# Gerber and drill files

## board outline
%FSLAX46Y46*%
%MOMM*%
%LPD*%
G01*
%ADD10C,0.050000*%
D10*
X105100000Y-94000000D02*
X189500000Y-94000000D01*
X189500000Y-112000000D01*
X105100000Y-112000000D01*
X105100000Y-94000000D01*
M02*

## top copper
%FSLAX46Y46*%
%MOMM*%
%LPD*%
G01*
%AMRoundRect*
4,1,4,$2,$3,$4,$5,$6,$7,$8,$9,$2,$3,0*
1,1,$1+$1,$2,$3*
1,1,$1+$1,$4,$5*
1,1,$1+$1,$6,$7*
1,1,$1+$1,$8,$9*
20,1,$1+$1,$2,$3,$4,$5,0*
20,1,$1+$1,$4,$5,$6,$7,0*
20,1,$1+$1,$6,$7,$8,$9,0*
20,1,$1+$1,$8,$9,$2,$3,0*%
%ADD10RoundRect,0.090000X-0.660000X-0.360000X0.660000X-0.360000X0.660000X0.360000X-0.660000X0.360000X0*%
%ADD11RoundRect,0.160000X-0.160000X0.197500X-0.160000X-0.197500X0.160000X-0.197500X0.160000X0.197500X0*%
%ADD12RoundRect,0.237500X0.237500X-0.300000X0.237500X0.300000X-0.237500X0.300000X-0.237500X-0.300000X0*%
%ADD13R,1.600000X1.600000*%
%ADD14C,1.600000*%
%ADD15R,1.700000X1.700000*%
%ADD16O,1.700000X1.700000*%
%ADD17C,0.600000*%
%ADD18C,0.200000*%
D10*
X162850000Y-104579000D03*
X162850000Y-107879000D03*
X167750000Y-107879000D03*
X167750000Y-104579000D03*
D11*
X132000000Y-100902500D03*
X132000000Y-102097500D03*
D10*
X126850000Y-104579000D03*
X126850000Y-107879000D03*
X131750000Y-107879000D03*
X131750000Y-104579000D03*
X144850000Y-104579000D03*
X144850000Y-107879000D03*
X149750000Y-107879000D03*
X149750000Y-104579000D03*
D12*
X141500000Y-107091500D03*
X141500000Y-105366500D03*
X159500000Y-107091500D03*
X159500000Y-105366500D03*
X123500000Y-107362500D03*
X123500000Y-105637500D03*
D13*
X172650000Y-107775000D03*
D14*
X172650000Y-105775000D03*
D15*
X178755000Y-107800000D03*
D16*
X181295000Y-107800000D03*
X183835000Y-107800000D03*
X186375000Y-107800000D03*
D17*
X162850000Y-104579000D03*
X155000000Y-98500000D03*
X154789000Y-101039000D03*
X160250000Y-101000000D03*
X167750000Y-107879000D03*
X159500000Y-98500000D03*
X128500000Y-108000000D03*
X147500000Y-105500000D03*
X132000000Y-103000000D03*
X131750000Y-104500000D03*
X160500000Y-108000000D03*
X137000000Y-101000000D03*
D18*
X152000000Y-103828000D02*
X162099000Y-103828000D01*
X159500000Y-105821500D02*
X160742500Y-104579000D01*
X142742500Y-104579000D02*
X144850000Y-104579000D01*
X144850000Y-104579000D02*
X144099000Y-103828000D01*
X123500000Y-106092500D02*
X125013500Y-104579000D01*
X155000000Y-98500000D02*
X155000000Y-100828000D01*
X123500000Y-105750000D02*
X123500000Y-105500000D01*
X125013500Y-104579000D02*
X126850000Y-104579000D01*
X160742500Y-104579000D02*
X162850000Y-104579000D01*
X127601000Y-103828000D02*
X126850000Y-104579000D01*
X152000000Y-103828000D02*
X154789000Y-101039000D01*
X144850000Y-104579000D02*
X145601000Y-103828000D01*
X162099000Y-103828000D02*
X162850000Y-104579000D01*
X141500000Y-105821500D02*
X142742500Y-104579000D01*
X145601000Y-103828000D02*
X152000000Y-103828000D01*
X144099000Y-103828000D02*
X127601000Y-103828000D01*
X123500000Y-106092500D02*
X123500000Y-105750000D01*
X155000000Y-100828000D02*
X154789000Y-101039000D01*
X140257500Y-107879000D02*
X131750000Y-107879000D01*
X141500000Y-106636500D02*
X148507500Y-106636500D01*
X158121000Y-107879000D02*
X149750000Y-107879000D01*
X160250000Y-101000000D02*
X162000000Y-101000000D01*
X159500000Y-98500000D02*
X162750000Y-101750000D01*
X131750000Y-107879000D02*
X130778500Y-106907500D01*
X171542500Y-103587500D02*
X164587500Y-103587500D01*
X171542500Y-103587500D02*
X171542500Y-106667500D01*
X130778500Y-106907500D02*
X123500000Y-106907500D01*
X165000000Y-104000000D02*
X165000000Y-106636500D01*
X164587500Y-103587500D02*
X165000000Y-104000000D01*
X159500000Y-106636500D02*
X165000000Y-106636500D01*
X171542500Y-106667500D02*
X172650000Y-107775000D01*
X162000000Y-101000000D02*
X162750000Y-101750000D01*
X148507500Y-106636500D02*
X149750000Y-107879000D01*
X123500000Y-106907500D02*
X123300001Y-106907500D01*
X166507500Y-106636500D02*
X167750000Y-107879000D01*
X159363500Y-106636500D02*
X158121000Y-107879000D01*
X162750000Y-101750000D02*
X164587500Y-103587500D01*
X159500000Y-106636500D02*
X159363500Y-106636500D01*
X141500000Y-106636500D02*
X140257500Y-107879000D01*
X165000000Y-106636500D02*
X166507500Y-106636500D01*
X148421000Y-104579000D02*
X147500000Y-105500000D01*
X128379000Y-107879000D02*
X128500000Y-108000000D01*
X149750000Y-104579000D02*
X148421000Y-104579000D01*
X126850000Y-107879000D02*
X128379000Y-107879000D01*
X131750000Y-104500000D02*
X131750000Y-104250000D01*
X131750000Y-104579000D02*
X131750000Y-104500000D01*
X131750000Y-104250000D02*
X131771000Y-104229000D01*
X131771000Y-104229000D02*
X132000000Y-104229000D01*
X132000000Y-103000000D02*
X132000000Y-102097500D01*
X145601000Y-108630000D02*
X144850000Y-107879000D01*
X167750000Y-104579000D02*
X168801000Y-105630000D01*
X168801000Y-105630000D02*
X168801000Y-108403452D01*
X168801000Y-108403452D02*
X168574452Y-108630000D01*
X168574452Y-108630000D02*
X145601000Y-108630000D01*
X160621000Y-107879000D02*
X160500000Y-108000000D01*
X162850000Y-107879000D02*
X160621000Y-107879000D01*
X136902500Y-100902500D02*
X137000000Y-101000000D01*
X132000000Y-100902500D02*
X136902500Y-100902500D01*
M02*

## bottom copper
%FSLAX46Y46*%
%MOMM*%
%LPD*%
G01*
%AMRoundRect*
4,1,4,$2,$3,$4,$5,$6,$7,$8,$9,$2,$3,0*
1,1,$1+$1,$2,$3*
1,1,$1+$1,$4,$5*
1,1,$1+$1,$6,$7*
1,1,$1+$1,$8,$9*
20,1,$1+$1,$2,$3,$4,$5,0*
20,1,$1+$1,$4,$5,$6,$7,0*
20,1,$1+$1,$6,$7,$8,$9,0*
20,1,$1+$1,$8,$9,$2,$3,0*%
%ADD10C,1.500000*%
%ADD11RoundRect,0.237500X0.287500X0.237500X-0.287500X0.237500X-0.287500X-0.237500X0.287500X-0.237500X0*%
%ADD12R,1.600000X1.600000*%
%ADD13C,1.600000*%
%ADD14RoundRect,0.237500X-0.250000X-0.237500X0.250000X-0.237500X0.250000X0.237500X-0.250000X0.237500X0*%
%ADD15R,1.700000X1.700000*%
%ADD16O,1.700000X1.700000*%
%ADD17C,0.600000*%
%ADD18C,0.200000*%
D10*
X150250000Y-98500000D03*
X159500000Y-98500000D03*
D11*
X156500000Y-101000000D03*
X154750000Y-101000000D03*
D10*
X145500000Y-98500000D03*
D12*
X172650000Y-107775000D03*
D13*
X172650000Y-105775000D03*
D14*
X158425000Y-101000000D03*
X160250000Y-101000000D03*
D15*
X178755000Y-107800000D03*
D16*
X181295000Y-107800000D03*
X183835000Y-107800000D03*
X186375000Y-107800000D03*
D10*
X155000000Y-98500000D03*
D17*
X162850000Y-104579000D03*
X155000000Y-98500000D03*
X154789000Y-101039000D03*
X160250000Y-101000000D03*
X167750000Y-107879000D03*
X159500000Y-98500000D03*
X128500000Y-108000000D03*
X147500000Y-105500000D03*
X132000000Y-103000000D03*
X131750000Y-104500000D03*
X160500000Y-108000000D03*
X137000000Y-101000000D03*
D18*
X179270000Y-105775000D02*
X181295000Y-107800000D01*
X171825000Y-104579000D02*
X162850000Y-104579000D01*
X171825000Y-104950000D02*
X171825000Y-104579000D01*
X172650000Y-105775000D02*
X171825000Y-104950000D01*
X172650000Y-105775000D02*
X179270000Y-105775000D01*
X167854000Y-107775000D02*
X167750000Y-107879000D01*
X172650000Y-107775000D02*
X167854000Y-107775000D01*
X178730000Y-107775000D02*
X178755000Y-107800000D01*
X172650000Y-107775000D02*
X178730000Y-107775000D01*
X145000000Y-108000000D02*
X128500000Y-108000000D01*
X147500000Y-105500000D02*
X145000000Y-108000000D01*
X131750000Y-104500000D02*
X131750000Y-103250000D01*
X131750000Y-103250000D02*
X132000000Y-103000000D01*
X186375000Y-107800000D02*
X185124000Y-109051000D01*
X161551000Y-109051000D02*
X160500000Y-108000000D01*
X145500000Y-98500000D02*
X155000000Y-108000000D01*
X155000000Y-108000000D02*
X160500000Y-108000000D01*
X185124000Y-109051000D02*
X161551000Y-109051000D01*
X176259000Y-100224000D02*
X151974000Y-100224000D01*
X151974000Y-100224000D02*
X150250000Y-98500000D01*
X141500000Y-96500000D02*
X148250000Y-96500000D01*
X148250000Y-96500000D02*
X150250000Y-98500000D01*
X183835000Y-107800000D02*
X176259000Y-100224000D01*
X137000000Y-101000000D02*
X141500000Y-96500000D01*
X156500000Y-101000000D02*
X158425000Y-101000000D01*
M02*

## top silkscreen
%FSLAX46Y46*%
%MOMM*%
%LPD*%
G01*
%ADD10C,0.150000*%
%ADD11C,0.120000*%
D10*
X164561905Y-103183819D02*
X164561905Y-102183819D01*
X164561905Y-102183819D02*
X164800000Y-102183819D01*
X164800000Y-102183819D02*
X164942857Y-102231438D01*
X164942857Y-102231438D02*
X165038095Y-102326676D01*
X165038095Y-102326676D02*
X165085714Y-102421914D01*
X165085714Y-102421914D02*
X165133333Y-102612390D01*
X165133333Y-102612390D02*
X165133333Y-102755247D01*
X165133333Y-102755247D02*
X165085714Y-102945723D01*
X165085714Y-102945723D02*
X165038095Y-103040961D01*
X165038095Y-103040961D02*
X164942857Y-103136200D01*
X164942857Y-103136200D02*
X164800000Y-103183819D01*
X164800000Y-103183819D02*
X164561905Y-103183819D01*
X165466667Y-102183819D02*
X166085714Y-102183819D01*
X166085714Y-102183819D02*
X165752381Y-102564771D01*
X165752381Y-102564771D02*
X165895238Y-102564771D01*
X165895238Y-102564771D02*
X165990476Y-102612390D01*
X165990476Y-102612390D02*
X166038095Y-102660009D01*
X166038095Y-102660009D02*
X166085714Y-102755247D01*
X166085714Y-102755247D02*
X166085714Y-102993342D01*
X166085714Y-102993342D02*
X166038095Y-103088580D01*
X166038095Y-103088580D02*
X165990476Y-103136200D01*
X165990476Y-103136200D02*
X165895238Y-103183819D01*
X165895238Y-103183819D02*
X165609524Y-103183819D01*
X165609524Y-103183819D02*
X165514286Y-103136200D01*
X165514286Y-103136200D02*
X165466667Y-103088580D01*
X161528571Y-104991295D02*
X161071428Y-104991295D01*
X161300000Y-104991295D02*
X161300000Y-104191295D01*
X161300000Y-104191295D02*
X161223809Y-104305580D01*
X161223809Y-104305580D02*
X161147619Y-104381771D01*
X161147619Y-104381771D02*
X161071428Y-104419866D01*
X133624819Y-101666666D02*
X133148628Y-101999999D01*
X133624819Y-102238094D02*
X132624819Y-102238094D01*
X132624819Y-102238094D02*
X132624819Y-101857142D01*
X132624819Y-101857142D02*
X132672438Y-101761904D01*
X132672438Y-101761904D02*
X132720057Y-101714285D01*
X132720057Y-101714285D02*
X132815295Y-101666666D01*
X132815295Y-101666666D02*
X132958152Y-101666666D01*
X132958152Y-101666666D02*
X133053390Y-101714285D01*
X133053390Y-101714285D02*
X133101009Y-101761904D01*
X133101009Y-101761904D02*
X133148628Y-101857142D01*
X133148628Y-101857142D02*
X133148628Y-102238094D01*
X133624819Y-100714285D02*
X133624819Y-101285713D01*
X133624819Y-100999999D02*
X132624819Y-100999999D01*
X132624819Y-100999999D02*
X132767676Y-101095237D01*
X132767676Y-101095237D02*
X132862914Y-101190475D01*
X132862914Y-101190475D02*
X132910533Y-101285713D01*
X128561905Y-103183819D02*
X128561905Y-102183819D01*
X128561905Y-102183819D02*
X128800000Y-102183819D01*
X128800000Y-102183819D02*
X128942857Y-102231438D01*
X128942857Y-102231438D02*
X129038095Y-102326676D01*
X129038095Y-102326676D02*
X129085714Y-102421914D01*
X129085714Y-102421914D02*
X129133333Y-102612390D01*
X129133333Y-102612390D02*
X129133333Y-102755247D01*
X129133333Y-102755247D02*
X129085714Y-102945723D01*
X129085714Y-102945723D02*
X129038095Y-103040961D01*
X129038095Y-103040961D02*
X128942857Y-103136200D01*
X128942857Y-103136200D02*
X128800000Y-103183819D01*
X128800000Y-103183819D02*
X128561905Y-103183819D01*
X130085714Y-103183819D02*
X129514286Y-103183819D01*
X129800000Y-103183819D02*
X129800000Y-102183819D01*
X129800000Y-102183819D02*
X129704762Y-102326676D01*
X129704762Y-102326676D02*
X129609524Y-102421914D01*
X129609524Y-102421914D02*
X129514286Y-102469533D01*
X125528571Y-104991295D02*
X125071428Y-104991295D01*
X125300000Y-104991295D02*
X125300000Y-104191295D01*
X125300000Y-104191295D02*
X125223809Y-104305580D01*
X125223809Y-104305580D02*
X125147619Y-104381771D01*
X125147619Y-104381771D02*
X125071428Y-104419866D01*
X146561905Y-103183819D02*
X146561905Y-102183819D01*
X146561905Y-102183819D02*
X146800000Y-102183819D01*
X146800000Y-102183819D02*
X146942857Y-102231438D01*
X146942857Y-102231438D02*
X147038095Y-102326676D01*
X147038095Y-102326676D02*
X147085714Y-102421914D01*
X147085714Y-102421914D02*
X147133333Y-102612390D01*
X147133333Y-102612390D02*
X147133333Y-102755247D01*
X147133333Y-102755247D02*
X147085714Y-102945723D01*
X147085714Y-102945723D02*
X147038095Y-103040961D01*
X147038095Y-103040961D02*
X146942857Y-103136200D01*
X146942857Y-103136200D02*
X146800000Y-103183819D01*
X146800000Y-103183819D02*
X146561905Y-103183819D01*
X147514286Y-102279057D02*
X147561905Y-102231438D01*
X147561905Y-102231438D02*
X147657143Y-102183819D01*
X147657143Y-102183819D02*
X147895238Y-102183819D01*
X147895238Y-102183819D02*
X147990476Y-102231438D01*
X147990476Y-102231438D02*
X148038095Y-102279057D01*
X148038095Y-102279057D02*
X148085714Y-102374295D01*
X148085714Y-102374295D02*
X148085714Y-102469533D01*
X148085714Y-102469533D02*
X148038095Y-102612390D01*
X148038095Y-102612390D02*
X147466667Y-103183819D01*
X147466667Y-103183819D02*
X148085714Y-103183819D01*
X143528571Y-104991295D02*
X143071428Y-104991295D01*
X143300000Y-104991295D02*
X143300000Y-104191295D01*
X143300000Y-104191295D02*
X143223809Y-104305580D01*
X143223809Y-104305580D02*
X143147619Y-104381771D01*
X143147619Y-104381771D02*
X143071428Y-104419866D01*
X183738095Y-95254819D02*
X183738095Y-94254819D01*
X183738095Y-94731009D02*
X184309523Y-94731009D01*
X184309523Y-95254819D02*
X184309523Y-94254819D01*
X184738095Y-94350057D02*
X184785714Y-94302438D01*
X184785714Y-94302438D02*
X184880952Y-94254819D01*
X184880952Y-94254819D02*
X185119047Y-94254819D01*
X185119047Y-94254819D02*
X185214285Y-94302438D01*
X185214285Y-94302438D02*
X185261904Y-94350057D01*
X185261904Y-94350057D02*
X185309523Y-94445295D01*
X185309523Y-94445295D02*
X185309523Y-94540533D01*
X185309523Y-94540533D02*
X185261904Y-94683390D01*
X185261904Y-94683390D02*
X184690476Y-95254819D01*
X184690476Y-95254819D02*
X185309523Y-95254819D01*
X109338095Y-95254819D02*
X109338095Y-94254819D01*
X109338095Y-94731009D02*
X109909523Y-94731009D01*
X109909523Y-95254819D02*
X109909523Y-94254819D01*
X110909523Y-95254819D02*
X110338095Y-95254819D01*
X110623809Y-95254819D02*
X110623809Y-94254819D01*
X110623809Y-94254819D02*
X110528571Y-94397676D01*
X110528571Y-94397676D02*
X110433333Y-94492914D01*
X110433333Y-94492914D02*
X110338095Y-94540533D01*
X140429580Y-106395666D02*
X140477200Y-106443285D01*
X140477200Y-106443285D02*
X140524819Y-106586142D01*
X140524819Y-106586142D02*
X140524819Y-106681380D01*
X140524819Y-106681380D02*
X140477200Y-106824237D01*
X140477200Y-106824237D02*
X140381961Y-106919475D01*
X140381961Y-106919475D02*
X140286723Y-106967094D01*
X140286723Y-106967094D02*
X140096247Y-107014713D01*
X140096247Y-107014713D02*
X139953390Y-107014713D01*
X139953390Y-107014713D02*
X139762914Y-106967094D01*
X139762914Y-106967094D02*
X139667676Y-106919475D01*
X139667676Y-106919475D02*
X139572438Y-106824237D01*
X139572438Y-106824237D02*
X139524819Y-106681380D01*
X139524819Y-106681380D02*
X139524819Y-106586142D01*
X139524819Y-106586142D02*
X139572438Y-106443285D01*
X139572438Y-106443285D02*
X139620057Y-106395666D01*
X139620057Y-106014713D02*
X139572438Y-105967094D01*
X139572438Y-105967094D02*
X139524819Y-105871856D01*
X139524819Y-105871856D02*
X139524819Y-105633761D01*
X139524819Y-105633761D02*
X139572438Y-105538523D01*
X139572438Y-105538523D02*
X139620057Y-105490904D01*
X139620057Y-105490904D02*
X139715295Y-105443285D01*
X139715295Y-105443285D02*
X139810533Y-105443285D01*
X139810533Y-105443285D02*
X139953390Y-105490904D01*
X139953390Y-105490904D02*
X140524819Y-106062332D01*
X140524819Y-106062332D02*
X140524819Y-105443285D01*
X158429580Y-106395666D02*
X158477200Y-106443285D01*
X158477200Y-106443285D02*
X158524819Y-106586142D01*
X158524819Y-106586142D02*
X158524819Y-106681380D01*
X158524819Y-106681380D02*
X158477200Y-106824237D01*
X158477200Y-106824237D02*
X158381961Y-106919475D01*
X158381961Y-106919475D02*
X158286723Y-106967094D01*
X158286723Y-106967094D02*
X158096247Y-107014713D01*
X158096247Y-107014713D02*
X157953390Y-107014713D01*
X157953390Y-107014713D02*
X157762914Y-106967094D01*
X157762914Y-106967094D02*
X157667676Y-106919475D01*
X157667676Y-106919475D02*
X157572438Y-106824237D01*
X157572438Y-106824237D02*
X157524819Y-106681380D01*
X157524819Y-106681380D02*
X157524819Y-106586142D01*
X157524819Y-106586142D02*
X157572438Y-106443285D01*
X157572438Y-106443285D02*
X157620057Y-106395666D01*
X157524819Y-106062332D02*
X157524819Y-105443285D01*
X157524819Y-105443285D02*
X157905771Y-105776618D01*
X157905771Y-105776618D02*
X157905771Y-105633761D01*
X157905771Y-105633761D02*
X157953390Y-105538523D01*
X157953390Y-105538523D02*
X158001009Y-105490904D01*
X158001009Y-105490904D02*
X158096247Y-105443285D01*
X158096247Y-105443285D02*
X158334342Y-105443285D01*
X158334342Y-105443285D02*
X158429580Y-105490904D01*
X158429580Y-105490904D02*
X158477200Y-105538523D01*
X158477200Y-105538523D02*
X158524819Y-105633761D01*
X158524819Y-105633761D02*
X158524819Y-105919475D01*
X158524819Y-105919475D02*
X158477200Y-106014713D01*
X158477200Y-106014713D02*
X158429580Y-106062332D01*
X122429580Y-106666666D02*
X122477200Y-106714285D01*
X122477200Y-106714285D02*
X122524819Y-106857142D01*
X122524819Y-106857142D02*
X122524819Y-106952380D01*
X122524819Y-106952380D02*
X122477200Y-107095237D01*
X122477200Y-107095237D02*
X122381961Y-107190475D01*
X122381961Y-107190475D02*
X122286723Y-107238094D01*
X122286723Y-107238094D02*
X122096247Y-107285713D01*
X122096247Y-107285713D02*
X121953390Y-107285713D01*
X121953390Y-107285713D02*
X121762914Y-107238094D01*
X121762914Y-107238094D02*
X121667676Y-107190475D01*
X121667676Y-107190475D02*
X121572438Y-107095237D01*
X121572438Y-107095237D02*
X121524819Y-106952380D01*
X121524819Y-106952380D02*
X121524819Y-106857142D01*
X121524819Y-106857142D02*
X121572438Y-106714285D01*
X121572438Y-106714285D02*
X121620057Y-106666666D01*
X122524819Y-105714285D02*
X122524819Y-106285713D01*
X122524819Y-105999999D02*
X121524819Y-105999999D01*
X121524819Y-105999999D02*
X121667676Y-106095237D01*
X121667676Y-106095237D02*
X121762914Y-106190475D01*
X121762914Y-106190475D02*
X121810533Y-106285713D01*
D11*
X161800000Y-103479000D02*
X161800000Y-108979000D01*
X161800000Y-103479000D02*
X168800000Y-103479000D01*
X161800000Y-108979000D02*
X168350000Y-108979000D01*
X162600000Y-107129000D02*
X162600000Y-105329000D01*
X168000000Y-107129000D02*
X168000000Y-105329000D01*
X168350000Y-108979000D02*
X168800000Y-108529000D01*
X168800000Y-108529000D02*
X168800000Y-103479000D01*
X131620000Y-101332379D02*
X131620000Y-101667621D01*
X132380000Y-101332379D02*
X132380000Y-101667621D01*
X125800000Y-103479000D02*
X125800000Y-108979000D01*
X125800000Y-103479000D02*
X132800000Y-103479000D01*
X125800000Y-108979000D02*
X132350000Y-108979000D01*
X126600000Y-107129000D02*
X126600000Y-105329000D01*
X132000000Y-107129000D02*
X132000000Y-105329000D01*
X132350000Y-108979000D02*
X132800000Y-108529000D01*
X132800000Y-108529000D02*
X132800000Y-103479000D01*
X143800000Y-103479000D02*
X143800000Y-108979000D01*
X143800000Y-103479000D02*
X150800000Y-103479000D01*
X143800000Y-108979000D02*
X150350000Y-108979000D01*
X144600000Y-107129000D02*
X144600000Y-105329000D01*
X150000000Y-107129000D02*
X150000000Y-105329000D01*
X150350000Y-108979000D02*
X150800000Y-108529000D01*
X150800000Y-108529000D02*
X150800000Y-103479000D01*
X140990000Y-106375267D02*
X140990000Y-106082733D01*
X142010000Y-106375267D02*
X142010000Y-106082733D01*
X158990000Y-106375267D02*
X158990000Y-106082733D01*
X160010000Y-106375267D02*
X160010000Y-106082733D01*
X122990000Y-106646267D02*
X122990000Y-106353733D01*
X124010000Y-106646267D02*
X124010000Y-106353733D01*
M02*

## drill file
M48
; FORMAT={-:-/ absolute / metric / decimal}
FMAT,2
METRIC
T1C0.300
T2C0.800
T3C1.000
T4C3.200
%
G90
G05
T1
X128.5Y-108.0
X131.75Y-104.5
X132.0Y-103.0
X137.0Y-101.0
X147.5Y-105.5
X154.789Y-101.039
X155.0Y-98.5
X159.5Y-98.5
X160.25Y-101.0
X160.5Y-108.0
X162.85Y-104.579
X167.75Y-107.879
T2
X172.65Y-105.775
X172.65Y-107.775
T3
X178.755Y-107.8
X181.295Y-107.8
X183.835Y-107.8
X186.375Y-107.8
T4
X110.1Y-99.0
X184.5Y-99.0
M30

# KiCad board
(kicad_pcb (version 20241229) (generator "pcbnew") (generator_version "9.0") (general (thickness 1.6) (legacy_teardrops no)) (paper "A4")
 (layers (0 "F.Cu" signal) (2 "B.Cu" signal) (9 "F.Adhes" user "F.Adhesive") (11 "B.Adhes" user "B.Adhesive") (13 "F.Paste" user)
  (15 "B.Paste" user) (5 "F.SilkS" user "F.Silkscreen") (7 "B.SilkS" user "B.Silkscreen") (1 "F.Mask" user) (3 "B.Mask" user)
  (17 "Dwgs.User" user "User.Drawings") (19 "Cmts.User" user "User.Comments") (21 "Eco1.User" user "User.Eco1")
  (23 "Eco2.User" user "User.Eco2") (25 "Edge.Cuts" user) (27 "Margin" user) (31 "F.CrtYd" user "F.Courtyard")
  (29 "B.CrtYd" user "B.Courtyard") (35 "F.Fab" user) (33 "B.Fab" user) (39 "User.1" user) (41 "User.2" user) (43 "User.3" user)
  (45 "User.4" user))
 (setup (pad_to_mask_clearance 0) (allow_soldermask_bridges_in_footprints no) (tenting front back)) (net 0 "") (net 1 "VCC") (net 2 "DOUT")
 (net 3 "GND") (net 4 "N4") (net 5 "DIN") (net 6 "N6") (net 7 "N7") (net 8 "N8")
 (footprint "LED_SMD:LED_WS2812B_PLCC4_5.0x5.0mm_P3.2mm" (layer "F.Cu") (at 165.3 106.229)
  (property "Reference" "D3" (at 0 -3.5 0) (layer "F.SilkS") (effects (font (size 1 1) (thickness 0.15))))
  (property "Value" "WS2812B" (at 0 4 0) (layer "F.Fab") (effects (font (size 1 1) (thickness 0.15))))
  (fp_line (start -3.5 -2.75) (end -3.5 2.75) (stroke (width 0.12) (type default)) (layer "F.SilkS"))
  (fp_line (start -3.5 -2.75) (end 3.5 -2.75) (stroke (width 0.12) (type solid)) (layer "F.SilkS"))
  (fp_line (start -3.5 2.75) (end 3.05 2.75) (stroke (width 0.12) (type solid)) (layer "F.SilkS"))
  (fp_line (start -2.7 0.9) (end -2.7 -0.9) (stroke (width 0.12) (type default)) (layer "F.SilkS"))
  (fp_line (start 2.7 0.9) (end 2.7 -0.9) (stroke (width 0.12) (type default)) (layer "F.SilkS"))
  (fp_line (start 3.05 2.75) (end 3.5 2.3) (stroke (width 0.12) (type default)) (layer "F.SilkS"))
  (fp_line (start 3.5 2.3) (end 3.5 -2.75) (stroke (width 0.12) (type default)) (layer "F.SilkS"))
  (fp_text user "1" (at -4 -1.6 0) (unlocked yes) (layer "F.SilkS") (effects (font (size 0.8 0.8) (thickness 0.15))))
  (pad "1" smd roundrect (at -2.45 -1.65) (size 1.5 0.9) (layers "F.Cu" "F.Mask" "F.Paste") (roundrect_rratio 0.1) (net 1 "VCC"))
  (pad "2" smd roundrect (at -2.45 1.65) (size 1.5 0.9) (layers "F.Cu" "F.Mask" "F.Paste") (roundrect_rratio 0.1) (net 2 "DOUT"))
  (pad "3" smd roundrect (at 2.45 1.65) (size 1.5 0.9) (layers "F.Cu" "F.Mask" "F.Paste") (roundrect_rratio 0.1) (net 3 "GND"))
  (pad "4" smd roundrect (at 2.45 -1.65) (size 1.5 0.9) (layers "F.Cu" "F.Mask" "F.Paste") (roundrect_rratio 0.1) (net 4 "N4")))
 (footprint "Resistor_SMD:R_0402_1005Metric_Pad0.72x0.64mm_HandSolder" (layer "F.Cu") (at 132 101.5 -90)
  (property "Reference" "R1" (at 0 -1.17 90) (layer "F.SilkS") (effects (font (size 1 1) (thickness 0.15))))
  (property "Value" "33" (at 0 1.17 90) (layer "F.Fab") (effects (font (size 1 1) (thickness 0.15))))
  (fp_line (start -0.167621 0.38) (end 0.167621 0.38) (stroke (width 0.12) (type solid)) (layer "F.SilkS"))
  (fp_line (start -0.167621 -0.38) (end 0.167621 -0.38) (stroke (width 0.12) (type solid)) (layer "F.SilkS"))
  (pad "1" smd roundrect (at -0.5975 0 270) (size 0.715 0.64) (layers "F.Cu" "F.Mask" "F.Paste") (roundrect_rratio 0.25) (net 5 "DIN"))
  (pad "2" smd roundrect (at 0.5975 0 270) (size 0.715 0.64) (layers "F.Cu" "F.Mask" "F.Paste") (roundrect_rratio 0.25) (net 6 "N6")))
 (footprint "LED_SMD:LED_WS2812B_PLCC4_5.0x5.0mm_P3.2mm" (layer "F.Cu") (at 129.3 106.229)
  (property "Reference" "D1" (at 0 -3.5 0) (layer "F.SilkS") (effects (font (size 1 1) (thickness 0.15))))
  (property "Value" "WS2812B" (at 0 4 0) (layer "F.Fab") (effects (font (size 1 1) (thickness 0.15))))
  (fp_line (start -3.5 -2.75) (end -3.5 2.75) (stroke (width 0.12) (type default)) (layer "F.SilkS"))
  (fp_line (start -3.5 -2.75) (end 3.5 -2.75) (stroke (width 0.12) (type solid)) (layer "F.SilkS"))
  (fp_line (start -3.5 2.75) (end 3.05 2.75) (stroke (width 0.12) (type solid)) (layer "F.SilkS"))
  (fp_line (start -2.7 0.9) (end -2.7 -0.9) (stroke (width 0.12) (type default)) (layer "F.SilkS"))
  (fp_line (start 2.7 0.9) (end 2.7 -0.9) (stroke (width 0.12) (type default)) (layer "F.SilkS"))
  (fp_line (start 3.05 2.75) (end 3.5 2.3) (stroke (width 0.12) (type default)) (layer "F.SilkS"))
  (fp_line (start 3.5 2.3) (end 3.5 -2.75) (stroke (width 0.12) (type default)) (layer "F.SilkS"))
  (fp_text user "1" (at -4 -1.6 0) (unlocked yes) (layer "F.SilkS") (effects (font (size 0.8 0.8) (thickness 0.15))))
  (pad "1" smd roundrect (at -2.45 -1.65) (size 1.5 0.9) (layers "F.Cu" "F.Mask" "F.Paste") (roundrect_rratio 0.1) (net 1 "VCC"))
  (pad "2" smd roundrect (at -2.45 1.65) (size 1.5 0.9) (layers "F.Cu" "F.Mask" "F.Paste") (roundrect_rratio 0.1) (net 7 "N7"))
  (pad "3" smd roundrect (at 2.45 1.65) (size 1.5 0.9) (layers "F.Cu" "F.Mask" "F.Paste") (roundrect_rratio 0.1) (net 3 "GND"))
  (pad "4" smd roundrect (at 2.45 -1.65) (size 1.5 0.9) (layers "F.Cu" "F.Mask" "F.Paste") (roundrect_rratio 0.1) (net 6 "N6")))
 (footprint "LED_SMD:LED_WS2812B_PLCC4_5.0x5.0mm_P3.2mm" (layer "F.Cu") (at 147.3 106.229)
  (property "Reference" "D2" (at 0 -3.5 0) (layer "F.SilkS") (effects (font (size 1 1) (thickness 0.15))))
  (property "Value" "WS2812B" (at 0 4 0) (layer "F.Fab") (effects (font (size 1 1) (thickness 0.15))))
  (fp_line (start -3.5 -2.75) (end -3.5 2.75) (stroke (width 0.12) (type default)) (layer "F.SilkS"))
  (fp_line (start -3.5 -2.75) (end 3.5 -2.75) (stroke (width 0.12) (type solid)) (layer "F.SilkS"))
  (fp_line (start -3.5 2.75) (end 3.05 2.75) (stroke (width 0.12) (type solid)) (layer "F.SilkS"))
  (fp_line (start -2.7 0.9) (end -2.7 -0.9) (stroke (width 0.12) (type default)) (layer "F.SilkS"))
  (fp_line (start 2.7 0.9) (end 2.7 -0.9) (stroke (width 0.12) (type default)) (layer "F.SilkS"))
  (fp_line (start 3.05 2.75) (end 3.5 2.3) (stroke (width 0.12) (type default)) (layer "F.SilkS"))
  (fp_line (start 3.5 2.3) (end 3.5 -2.75) (stroke (width 0.12) (type default)) (layer "F.SilkS"))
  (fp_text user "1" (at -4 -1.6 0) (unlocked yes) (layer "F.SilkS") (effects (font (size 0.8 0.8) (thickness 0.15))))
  (pad "1" smd roundrect (at -2.45 -1.65) (size 1.5 0.9) (layers "F.Cu" "F.Mask" "F.Paste") (roundrect_rratio 0.1) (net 1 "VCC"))
  (pad "2" smd roundrect (at -2.45 1.65) (size 1.5 0.9) (layers "F.Cu" "F.Mask" "F.Paste") (roundrect_rratio 0.1) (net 4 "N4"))
  (pad "3" smd roundrect (at 2.45 1.65) (size 1.5 0.9) (layers "F.Cu" "F.Mask" "F.Paste") (roundrect_rratio 0.1) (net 3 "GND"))
  (pad "4" smd roundrect (at 2.45 -1.65) (size 1.5 0.9) (layers "F.Cu" "F.Mask" "F.Paste") (roundrect_rratio 0.1) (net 7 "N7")))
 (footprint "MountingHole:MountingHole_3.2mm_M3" (layer "F.Cu") (at 184.5 99)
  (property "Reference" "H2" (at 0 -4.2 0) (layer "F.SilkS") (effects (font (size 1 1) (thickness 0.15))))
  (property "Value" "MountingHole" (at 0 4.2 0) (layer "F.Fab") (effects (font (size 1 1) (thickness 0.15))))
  (pad "" np_thru_hole circle (at 0 0) (size 3.2 3.2) (drill 3.2) (layers "*.Cu" "*.Mask")))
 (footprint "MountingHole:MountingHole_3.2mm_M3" (layer "F.Cu") (at 110.1 99)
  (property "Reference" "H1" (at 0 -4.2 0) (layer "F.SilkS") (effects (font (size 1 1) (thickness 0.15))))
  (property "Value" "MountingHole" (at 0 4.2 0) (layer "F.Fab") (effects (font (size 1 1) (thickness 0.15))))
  (pad "" np_thru_hole circle (at 0 0) (size 3.2 3.2) (drill 3.2) (layers "*.Cu" "*.Mask")))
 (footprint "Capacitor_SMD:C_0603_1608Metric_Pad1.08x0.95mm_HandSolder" (layer "F.Cu") (at 141.5 106.229 90)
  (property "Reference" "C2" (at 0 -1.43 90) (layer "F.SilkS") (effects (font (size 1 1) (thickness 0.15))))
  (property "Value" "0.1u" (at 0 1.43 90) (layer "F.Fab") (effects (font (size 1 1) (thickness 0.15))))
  (fp_line (start -0.146267 -0.51) (end 0.146267 -0.51) (stroke (width 0.12) (type solid)) (layer "F.SilkS"))
  (fp_line (start -0.146267 0.51) (end 0.146267 0.51) (stroke (width 0.12) (type solid)) (layer "F.SilkS"))
  (pad "1" smd roundrect (at -0.8625 0 90) (size 1.075 0.95) (layers "F.Cu" "F.Mask" "F.Paste") (roundrect_rratio 0.25) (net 3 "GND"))
  (pad "2" smd roundrect (at 0.8625 0 90) (size 1.075 0.95) (layers "F.Cu" "F.Mask" "F.Paste") (roundrect_rratio 0.25) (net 1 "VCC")))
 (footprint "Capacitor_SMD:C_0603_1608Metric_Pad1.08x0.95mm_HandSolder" (layer "F.Cu") (at 159.5 106.229 90)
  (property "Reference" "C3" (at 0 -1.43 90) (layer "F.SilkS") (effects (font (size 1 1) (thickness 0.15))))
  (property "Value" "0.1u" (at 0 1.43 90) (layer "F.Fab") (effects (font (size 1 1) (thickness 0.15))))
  (fp_line (start -0.146267 -0.51) (end 0.146267 -0.51) (stroke (width 0.12) (type solid)) (layer "F.SilkS"))
  (fp_line (start -0.146267 0.51) (end 0.146267 0.51) (stroke (width 0.12) (type solid)) (layer "F.SilkS"))
  (pad "1" smd roundrect (at -0.8625 0 90) (size 1.075 0.95) (layers "F.Cu" "F.Mask" "F.Paste") (roundrect_rratio 0.25) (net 3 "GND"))
  (pad "2" smd roundrect (at 0.8625 0 90) (size 1.075 0.95) (layers "F.Cu" "F.Mask" "F.Paste") (roundrect_rratio 0.25) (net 1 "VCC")))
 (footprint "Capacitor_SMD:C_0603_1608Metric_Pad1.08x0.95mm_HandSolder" (layer "F.Cu") (at 123.5 106.5 90)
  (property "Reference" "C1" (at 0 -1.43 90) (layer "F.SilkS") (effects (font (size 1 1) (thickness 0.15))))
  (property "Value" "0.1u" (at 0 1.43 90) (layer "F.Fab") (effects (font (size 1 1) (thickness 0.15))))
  (fp_line (start -0.146267 -0.51) (end 0.146267 -0.51) (stroke (width 0.12) (type solid)) (layer "F.SilkS"))
  (fp_line (start -0.146267 0.51) (end 0.146267 0.51) (stroke (width 0.12) (type solid)) (layer "F.SilkS"))
  (pad "1" smd roundrect (at -0.8625 0 90) (size 1.075 0.95) (layers "F.Cu" "F.Mask" "F.Paste") (roundrect_rratio 0.25) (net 3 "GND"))
  (pad "2" smd roundrect (at 0.8625 0 90) (size 1.075 0.95) (layers "F.Cu" "F.Mask" "F.Paste") (roundrect_rratio 0.25) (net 1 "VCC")))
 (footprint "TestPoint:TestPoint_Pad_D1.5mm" (layer "B.Cu") (at 150.25 98.5 180)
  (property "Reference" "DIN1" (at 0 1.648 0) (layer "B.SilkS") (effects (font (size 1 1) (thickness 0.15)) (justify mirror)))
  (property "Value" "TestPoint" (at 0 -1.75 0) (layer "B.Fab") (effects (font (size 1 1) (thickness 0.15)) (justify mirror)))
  (pad "1" smd circle (at 0 0 180) (size 1.5 1.5) (layers "B.Cu" "B.Mask") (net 5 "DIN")))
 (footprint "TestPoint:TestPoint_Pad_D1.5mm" (layer "B.Cu") (at 159.5 98.5 180)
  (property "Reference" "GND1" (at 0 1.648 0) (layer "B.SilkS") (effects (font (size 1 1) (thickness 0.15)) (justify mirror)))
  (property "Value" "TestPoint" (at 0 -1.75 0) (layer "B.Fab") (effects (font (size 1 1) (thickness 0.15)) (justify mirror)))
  (pad "1" smd circle (at 0 0 180) (size 1.5 1.5) (layers "B.Cu" "B.Mask") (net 3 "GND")))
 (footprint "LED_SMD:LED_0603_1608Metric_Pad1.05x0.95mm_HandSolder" (layer "B.Cu") (at 155.625 101 180)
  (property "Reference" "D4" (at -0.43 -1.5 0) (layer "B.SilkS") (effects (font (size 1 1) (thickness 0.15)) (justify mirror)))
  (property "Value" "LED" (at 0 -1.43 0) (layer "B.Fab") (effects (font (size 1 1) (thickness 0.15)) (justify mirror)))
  (pad "1" smd roundrect (at -0.875 0 180) (size 1.05 0.95) (layers "B.Cu" "B.Mask" "B.Paste") (roundrect_rratio 0.25) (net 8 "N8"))
  (pad "2" smd roundrect (at 0.875 0 180) (size 1.05 0.95) (layers "B.Cu" "B.Mask" "B.Paste") (roundrect_rratio 0.25) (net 1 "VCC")))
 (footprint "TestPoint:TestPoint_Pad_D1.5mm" (layer "B.Cu") (at 145.5 98.5 180)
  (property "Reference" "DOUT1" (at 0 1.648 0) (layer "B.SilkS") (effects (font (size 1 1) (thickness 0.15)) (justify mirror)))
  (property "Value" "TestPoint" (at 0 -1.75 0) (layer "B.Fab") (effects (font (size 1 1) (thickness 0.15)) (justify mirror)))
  (pad "1" smd circle (at 0 0 180) (size 1.5 1.5) (layers "B.Cu" "B.Mask") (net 2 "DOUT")))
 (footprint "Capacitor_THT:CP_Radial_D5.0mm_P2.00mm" (layer "B.Cu") (at 172.65 107.775 90)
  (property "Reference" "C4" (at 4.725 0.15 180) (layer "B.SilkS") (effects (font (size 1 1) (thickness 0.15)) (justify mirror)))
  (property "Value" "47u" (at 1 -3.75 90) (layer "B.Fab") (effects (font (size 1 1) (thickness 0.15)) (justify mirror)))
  (pad "1" thru_hole rect (at 0 0 90) (size 1.6 1.6) (drill 0.8) (layers "*.Cu" "*.Mask") (remove_unused_layers no) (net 3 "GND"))
  (pad "2" thru_hole circle (at 2 0 90) (size 1.6 1.6) (drill 0.8) (layers "*.Cu" "*.Mask") (remove_unused_layers no) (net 1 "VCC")))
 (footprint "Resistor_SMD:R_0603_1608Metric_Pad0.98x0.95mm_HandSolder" (layer "B.Cu") (at 159.3375 101)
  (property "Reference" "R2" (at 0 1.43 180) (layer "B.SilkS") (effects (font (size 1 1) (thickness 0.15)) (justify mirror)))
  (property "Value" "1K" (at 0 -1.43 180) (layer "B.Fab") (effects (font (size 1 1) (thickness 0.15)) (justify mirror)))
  (pad "1" smd roundrect (at -0.9125 0) (size 0.975 0.95) (layers "B.Cu" "B.Mask" "B.Paste") (roundrect_rratio 0.25) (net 8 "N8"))
  (pad "2" smd roundrect (at 0.9125 0) (size 0.975 0.95) (layers "B.Cu" "B.Mask" "B.Paste") (roundrect_rratio 0.25) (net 3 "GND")))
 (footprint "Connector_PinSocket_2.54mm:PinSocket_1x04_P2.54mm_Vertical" (layer "B.Cu") (at 178.755 107.8 -90)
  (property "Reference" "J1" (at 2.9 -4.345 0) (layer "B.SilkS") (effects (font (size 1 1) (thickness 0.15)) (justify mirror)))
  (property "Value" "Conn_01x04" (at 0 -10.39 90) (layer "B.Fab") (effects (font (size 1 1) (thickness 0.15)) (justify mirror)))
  (pad "1" thru_hole rect (at 0 0 270) (size 1.7 1.7) (drill 1) (layers "*.Cu" "*.Mask") (remove_unused_layers no) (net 3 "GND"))
  (pad "2" thru_hole oval (at 0 -2.54 270) (size 1.7 1.7) (drill 1) (layers "*.Cu" "*.Mask") (remove_unused_layers no) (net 1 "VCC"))
  (pad "3" thru_hole oval (at 0 -5.08 270) (size 1.7 1.7) (drill 1) (layers "*.Cu" "*.Mask") (remove_unused_layers no) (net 5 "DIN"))
  (pad "4" thru_hole oval (at 0 -7.62 270) (size 1.7 1.7) (drill 1) (layers "*.Cu" "*.Mask") (remove_unused_layers no) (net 2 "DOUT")))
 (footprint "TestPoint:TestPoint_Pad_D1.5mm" (layer "B.Cu") (at 155 98.5 180)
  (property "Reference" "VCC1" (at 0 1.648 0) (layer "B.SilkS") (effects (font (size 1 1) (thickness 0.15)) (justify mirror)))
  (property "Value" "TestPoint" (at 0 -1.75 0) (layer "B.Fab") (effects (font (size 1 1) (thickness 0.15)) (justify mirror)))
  (pad "1" smd circle (at 0 0 180) (size 1.5 1.5) (layers "B.Cu" "B.Mask") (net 1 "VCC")))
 (gr_rect (start 105.1 94) (end 189.5 112) (stroke (width 0.05) (type solid)) (fill no) (layer "Edge.Cuts"))
 (segment (start 152 103.828) (end 162.099 103.828) (width 0.2) (layer "F.Cu") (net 1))
 (segment (start 159.5 105.8215) (end 160.7425 104.579) (width 0.2) (layer "F.Cu") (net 1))
 (segment (start 142.7425 104.579) (end 144.85 104.579) (width 0.2) (layer "F.Cu") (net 1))
 (segment (start 144.85 104.579) (end 144.099 103.828) (width 0.2) (layer "F.Cu") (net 1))
 (segment (start 123.5 106.0925) (end 125.0135 104.579) (width 0.2) (layer "F.Cu") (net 1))
 (segment (start 155 98.5) (end 155 100.828) (width 0.2) (layer "F.Cu") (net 1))
 (segment (start 123.5 105.75) (end 123.5 105.5) (width 0.2) (layer "F.Cu") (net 1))
 (segment (start 125.0135 104.579) (end 126.85 104.579) (width 0.2) (layer "F.Cu") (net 1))
 (segment (start 160.7425 104.579) (end 162.85 104.579) (width 0.2) (layer "F.Cu") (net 1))
 (segment (start 127.601 103.828) (end 126.85 104.579) (width 0.2) (layer "F.Cu") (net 1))
 (segment (start 152 103.828) (end 154.789 101.039) (width 0.2) (layer "F.Cu") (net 1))
 (segment (start 144.85 104.579) (end 145.601 103.828) (width 0.2) (layer "F.Cu") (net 1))
 (segment (start 162.099 103.828) (end 162.85 104.579) (width 0.2) (layer "F.Cu") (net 1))
 (segment (start 141.5 105.8215) (end 142.7425 104.579) (width 0.2) (layer "F.Cu") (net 1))
 (segment (start 145.601 103.828) (end 152 103.828) (width 0.2) (layer "F.Cu") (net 1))
 (segment (start 144.099 103.828) (end 127.601 103.828) (width 0.2) (layer "F.Cu") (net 1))
 (segment (start 123.5 106.0925) (end 123.5 105.75) (width 0.2) (layer "F.Cu") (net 1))
 (segment (start 155 100.828) (end 154.789 101.039) (width 0.2) (layer "F.Cu") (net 1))
 (via (at 162.85 104.579) (size 0.6) (drill 0.3) (layers "F.Cu" "B.Cu") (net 1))
 (via (at 155 98.5) (size 0.6) (drill 0.3) (layers "F.Cu" "B.Cu") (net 1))
 (via (at 154.789 101.039) (size 0.6) (drill 0.3) (layers "F.Cu" "B.Cu") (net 1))
 (segment (start 179.27 105.775) (end 181.295 107.8) (width 0.2) (layer "B.Cu") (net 1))
 (segment (start 171.825 104.579) (end 162.85 104.579) (width 0.2) (layer "B.Cu") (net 1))
 (segment (start 171.825 104.95) (end 171.825 104.579) (width 0.2) (layer "B.Cu") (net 1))
 (segment (start 172.65 105.775) (end 171.825 104.95) (width 0.2) (layer "B.Cu") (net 1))
 (segment (start 172.65 105.775) (end 179.27 105.775) (width 0.2) (layer "B.Cu") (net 1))
 (segment (start 140.2575 107.879) (end 131.75 107.879) (width 0.2) (layer "F.Cu") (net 3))
 (segment (start 141.5 106.6365) (end 148.5075 106.6365) (width 0.2) (layer "F.Cu") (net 3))
 (segment (start 158.121 107.879) (end 149.75 107.879) (width 0.2) (layer "F.Cu") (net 3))
 (segment (start 160.25 101) (end 162 101) (width 0.2) (layer "F.Cu") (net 3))
 (segment (start 159.5 98.5) (end 162.75 101.75) (width 0.2) (layer "F.Cu") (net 3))
 (segment (start 131.75 107.879) (end 130.7785 106.9075) (width 0.2) (layer "F.Cu") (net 3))
 (segment (start 171.5425 103.5875) (end 164.5875 103.5875) (width 0.2) (layer "F.Cu") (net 3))
 (segment (start 171.5425 103.5875) (end 171.5425 106.6675) (width 0.2) (layer "F.Cu") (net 3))
 (segment (start 130.7785 106.9075) (end 123.5 106.9075) (width 0.2) (layer "F.Cu") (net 3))
 (segment (start 165 104) (end 165 106.6365) (width 0.2) (layer "F.Cu") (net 3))
 (segment (start 164.5875 103.5875) (end 165 104) (width 0.2) (layer "F.Cu") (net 3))
 (segment (start 159.5 106.6365) (end 165 106.6365) (width 0.2) (layer "F.Cu") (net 3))
 (segment (start 171.5425 106.6675) (end 172.65 107.775) (width 0.2) (layer "F.Cu") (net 3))
 (segment (start 162 101) (end 162.75 101.75) (width 0.2) (layer "F.Cu") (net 3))
 (segment (start 148.5075 106.6365) (end 149.75 107.879) (width 0.2) (layer "F.Cu") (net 3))
 (segment (start 123.5 106.9075) (end 123.300001 106.9075) (width 0.2) (layer "F.Cu") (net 3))
 (segment (start 166.5075 106.6365) (end 167.75 107.879) (width 0.2) (layer "F.Cu") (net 3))
 (segment (start 159.3635 106.6365) (end 158.121 107.879) (width 0.2) (layer "F.Cu") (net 3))
 (segment (start 162.75 101.75) (end 164.5875 103.5875) (width 0.2) (layer "F.Cu") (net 3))
 (segment (start 159.5 106.6365) (end 159.3635 106.6365) (width 0.2) (layer "F.Cu") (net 3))
 (segment (start 141.5 106.6365) (end 140.2575 107.879) (width 0.2) (layer "F.Cu") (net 3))
 (segment (start 165 106.6365) (end 166.5075 106.6365) (width 0.2) (layer "F.Cu") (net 3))
 (via (at 160.25 101) (size 0.6) (drill 0.3) (layers "F.Cu" "B.Cu") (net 3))
 (via (at 167.75 107.879) (size 0.6) (drill 0.3) (layers "F.Cu" "B.Cu") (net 3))
 (via (at 159.5 98.5) (size 0.6) (drill 0.3) (layers "F.Cu" "B.Cu") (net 3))
 (segment (start 167.854 107.775) (end 167.75 107.879) (width 0.2) (layer "B.Cu") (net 3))
 (segment (start 172.65 107.775) (end 167.854 107.775) (width 0.2) (layer "B.Cu") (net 3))
 (segment (start 178.73 107.775) (end 178.755 107.8) (width 0.2) (layer "B.Cu") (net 3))
 (segment (start 172.65 107.775) (end 178.73 107.775) (width 0.2) (layer "B.Cu") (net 3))
 (segment (start 148.421 104.579) (end 147.5 105.5) (width 0.2) (layer "F.Cu") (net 7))
 (segment (start 128.379 107.879) (end 128.5 108) (width 0.2) (layer "F.Cu") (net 7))
 (segment (start 149.75 104.579) (end 148.421 104.579) (width 0.2) (layer "F.Cu") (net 7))
 (segment (start 126.85 107.879) (end 128.379 107.879) (width 0.2) (layer "F.Cu") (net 7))
 (via (at 128.5 108) (size 0.6) (drill 0.3) (layers "F.Cu" "B.Cu") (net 7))
 (via (at 147.5 105.5) (size 0.6) (drill 0.3) (layers "F.Cu" "B.Cu") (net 7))
 (segment (start 145 108) (end 128.5 108) (width 0.2) (layer "B.Cu") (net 7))
 (segment (start 147.5 105.5) (end 145 108) (width 0.2) (layer "B.Cu") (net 7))
 (segment (start 131.75 104.5) (end 131.75 104.25) (width 0.2) (layer "F.Cu") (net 6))
 (segment (start 131.75 104.579) (end 131.75 104.5) (width 0.2) (layer "F.Cu") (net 6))
 (segment (start 131.75 104.25) (end 131.771 104.229) (width 0.2) (layer "F.Cu") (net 6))
 (segment (start 131.771 104.229) (end 132 104.229) (width 0.2) (layer "F.Cu") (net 6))
 (segment (start 132 103) (end 132 102.0975) (width 0.2) (layer "F.Cu") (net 6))
 (via (at 132 103) (size 0.6) (drill 0.3) (layers "F.Cu" "B.Cu") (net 6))
 (via (at 131.75 104.5) (size 0.6) (drill 0.3) (layers "F.Cu" "B.Cu") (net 6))
 (segment (start 131.75 104.5) (end 131.75 103.25) (width 0.2) (layer "B.Cu") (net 6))
 (segment (start 131.75 103.25) (end 132 103) (width 0.2) (layer "B.Cu") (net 6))
 (segment (start 145.601 108.63) (end 144.85 107.879) (width 0.2) (layer "F.Cu") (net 4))
 (segment (start 167.75 104.579) (end 168.801 105.63) (width 0.2) (layer "F.Cu") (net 4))
 (segment (start 168.801 105.63) (end 168.801 108.403452) (width 0.2) (layer "F.Cu") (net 4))
 (segment (start 168.801 108.403452) (end 168.574452 108.63) (width 0.2) (layer "F.Cu") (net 4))
 (segment (start 168.574452 108.63) (end 145.601 108.63) (width 0.2) (layer "F.Cu") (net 4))
 (segment (start 160.621 107.879) (end 160.5 108) (width 0.2) (layer "F.Cu") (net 2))
 (segment (start 162.85 107.879) (end 160.621 107.879) (width 0.2) (layer "F.Cu") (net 2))
 (via (at 160.5 108) (size 0.6) (drill 0.3) (layers "F.Cu" "B.Cu") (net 2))
 (segment (start 186.375 107.8) (end 185.124 109.051) (width 0.2) (layer "B.Cu") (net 2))
 (segment (start 161.551 109.051) (end 160.5 108) (width 0.2) (layer "B.Cu") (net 2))
 (segment (start 145.5 98.5) (end 155 108) (width 0.2) (layer "B.Cu") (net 2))
 (segment (start 155 108) (end 160.5 108) (width 0.2) (layer "B.Cu") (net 2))
 (segment (start 185.124 109.051) (end 161.551 109.051) (width 0.2) (layer "B.Cu") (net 2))
 (segment (start 136.9025 100.9025) (end 137 101) (width 0.2) (layer "F.Cu") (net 5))
 (segment (start 132 100.9025) (end 136.9025 100.9025) (width 0.2) (layer "F.Cu") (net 5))
 (via (at 137 101) (size 0.6) (drill 0.3) (layers "F.Cu" "B.Cu") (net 5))
 (segment (start 176.259 100.224) (end 151.974 100.224) (width 0.2) (layer "B.Cu") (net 5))
 (segment (start 151.974 100.224) (end 150.25 98.5) (width 0.2) (layer "B.Cu") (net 5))
 (segment (start 141.5 96.5) (end 148.25 96.5) (width 0.2) (layer "B.Cu") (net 5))
 (segment (start 148.25 96.5) (end 150.25 98.5) (width 0.2) (layer "B.Cu") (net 5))
 (segment (start 183.835 107.8) (end 176.259 100.224) (width 0.2) (layer "B.Cu") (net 5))
 (segment (start 137 101) (end 141.5 96.5) (width 0.2) (layer "B.Cu") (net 5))
 (segment (start 156.5 101) (end 158.425 101) (width 0.2) (layer "B.Cu") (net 8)))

